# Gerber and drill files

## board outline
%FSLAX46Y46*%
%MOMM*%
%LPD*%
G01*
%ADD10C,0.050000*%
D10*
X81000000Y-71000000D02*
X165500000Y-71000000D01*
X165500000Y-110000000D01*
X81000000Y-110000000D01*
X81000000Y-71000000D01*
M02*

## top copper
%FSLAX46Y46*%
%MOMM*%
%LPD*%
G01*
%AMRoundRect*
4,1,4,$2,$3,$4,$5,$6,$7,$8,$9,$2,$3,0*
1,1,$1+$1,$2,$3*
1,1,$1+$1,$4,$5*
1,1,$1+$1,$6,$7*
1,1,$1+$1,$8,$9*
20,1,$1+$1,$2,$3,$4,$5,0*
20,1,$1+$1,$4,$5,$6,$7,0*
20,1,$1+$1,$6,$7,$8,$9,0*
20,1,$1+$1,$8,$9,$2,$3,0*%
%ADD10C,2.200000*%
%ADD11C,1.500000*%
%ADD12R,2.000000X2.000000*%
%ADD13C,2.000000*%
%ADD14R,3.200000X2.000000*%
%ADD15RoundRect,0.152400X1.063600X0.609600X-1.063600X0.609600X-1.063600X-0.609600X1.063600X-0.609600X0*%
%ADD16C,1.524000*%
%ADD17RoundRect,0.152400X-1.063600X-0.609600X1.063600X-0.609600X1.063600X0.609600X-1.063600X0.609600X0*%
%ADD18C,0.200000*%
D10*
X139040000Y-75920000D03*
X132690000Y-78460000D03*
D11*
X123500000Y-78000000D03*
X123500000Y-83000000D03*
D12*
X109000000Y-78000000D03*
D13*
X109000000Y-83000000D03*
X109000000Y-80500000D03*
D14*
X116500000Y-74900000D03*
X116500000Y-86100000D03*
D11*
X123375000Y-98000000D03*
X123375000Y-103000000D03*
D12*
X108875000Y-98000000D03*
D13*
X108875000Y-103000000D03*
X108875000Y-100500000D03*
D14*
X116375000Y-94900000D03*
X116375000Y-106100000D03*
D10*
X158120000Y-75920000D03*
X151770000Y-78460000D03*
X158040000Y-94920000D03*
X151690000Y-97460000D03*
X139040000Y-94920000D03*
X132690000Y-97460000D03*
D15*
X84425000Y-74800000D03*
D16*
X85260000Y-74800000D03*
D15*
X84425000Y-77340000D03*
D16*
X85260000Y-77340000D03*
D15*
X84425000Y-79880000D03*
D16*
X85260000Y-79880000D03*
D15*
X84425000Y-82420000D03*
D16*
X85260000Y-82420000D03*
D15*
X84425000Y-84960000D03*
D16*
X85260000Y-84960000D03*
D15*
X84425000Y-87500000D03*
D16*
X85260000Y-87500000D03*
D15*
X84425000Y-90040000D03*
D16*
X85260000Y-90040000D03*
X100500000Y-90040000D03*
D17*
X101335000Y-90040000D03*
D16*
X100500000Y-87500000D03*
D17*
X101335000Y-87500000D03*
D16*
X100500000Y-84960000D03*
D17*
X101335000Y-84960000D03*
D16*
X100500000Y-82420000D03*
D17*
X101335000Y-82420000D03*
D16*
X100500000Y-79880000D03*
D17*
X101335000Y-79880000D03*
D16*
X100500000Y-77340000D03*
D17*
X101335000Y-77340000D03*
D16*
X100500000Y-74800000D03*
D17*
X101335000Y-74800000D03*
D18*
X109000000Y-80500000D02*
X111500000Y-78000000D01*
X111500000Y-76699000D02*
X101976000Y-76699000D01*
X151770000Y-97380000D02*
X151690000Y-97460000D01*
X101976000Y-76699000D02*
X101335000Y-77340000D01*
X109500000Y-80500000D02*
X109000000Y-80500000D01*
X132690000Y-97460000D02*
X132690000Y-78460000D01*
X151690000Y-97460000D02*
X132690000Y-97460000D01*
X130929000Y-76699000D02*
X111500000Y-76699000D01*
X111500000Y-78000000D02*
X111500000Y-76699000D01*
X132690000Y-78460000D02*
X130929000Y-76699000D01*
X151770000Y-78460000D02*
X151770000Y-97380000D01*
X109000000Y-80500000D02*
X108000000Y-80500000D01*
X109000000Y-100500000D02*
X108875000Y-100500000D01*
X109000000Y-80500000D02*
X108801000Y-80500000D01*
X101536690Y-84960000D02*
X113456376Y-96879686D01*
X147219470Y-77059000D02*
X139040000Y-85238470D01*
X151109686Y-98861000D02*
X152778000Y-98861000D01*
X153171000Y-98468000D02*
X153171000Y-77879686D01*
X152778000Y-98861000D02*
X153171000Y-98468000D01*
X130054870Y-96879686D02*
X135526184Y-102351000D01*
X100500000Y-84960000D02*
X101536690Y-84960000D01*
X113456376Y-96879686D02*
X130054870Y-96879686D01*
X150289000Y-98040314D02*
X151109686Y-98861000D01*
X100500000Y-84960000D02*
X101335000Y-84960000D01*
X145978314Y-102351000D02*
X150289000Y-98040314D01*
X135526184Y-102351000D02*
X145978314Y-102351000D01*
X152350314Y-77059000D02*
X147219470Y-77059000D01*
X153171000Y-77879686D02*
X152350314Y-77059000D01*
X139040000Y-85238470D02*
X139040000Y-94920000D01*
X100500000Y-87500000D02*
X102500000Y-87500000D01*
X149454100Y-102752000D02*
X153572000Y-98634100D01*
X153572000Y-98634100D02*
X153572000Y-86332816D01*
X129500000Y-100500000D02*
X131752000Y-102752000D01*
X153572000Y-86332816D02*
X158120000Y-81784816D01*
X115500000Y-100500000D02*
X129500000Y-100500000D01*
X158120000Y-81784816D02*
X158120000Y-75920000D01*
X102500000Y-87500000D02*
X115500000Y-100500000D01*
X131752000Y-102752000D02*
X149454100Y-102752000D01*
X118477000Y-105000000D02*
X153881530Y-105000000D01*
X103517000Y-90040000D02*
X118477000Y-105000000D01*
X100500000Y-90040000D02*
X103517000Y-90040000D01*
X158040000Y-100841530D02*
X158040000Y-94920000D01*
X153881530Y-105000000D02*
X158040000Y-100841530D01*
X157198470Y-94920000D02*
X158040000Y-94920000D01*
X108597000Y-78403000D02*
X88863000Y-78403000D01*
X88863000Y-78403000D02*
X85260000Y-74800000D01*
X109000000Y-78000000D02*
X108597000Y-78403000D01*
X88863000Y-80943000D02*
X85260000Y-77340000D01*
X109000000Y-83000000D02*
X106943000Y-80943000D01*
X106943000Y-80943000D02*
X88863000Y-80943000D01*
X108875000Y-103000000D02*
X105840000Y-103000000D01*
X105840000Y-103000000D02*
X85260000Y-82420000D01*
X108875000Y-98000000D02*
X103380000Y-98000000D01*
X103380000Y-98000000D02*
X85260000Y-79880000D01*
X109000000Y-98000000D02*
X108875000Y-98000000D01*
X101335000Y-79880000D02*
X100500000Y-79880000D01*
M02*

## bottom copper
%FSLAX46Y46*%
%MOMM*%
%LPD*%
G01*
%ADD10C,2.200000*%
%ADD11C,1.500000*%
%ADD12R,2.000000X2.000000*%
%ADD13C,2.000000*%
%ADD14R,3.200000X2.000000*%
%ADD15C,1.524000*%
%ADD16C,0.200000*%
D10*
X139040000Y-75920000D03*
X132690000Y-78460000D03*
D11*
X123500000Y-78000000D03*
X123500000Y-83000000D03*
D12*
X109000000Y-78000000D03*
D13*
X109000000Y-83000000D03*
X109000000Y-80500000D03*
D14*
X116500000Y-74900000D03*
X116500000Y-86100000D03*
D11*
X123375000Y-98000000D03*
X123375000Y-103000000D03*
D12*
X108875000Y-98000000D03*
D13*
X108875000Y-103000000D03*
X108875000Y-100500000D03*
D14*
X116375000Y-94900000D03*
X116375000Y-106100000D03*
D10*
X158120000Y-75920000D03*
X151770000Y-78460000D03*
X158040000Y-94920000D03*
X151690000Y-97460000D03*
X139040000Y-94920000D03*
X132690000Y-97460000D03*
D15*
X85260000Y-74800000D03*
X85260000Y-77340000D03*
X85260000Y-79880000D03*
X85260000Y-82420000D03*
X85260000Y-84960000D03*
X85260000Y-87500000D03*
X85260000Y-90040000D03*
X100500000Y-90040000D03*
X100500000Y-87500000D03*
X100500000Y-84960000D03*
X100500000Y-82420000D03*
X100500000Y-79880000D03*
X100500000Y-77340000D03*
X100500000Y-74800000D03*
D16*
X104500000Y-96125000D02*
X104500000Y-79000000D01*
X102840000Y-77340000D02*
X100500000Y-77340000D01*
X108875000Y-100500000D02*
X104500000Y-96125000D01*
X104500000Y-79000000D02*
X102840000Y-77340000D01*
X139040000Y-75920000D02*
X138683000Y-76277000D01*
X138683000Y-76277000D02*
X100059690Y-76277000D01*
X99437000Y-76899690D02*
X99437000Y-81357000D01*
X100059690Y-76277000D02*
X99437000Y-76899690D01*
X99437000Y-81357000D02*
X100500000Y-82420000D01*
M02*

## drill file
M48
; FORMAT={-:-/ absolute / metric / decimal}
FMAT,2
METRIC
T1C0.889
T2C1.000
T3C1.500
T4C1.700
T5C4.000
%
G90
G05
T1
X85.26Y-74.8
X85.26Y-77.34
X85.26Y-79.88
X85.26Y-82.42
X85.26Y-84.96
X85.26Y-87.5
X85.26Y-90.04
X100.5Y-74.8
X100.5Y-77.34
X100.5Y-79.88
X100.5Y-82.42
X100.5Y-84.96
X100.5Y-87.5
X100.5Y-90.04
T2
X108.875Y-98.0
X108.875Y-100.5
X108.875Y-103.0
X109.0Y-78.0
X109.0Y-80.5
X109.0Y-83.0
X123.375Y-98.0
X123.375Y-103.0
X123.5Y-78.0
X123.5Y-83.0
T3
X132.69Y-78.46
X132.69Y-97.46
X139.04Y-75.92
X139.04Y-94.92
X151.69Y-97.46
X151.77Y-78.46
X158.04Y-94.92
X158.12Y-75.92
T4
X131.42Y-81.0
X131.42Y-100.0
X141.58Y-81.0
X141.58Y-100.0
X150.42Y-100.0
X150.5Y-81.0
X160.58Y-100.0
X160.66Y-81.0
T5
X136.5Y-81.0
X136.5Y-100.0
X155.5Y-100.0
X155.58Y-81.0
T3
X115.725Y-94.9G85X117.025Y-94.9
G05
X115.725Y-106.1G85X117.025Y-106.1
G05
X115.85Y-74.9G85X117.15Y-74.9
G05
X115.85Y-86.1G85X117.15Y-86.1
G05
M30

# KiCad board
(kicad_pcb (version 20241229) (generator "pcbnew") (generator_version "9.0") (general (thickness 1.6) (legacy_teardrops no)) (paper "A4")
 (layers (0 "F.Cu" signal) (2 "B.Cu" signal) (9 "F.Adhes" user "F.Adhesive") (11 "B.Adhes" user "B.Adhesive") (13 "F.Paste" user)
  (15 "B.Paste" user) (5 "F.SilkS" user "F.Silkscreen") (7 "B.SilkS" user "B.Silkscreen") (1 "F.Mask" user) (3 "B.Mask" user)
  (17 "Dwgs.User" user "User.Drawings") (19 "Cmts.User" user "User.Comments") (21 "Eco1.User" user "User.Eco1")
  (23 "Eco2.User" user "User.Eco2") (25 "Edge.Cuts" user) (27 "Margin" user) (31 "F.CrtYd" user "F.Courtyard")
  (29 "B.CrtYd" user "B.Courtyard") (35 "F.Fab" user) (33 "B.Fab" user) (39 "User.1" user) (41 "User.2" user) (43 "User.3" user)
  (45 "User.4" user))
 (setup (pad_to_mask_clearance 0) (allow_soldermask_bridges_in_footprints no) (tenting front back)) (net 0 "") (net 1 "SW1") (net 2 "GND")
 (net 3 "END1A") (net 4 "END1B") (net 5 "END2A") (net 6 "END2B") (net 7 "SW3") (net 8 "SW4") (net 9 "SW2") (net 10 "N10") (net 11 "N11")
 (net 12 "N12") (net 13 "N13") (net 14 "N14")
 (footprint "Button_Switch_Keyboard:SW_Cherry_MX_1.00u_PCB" (layer "F.Cu") (at 139.04 75.92)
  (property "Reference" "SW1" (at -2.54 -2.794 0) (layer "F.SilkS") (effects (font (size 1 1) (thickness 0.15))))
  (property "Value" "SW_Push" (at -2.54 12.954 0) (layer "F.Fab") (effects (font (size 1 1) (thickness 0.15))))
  (pad "" np_thru_hole circle (at -7.62 5.08) (size 1.7 1.7) (drill 1.7) (layers "*.Cu" "*.Mask"))
  (pad "" np_thru_hole circle (at -2.54 5.08) (size 4 4) (drill 4) (layers "*.Cu" "*.Mask"))
  (pad "" np_thru_hole circle (at 2.54 5.08) (size 1.7 1.7) (drill 1.7) (layers "*.Cu" "*.Mask"))
  (pad "1" thru_hole circle (at 0 0) (size 2.2 2.2) (drill 1.5) (layers "*.Cu" "*.Mask") (remove_unused_layers no) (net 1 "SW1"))
  (pad "2" thru_hole circle (at -6.35 2.54) (size 2.2 2.2) (drill 1.5) (layers "*.Cu" "*.Mask") (remove_unused_layers no) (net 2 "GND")))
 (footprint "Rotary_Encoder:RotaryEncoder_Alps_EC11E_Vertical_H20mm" (layer "F.Cu") (at 109 78)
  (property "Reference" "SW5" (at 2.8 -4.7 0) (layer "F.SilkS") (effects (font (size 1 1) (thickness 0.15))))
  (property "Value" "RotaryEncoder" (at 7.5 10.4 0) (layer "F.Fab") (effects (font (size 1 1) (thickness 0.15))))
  (pad "" thru_hole circle (at 14.5 0) (size 1.5 1.5) (drill 1) (layers "*.Cu" "*.Mask") (remove_unused_layers no))
  (pad "" thru_hole circle (at 14.5 5) (size 1.5 1.5) (drill 1) (layers "*.Cu" "*.Mask") (remove_unused_layers no))
  (pad "A" thru_hole rect (at 0 0) (size 2 2) (drill 1) (layers "*.Cu" "*.Mask") (remove_unused_layers no) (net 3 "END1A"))
  (pad "B" thru_hole circle (at 0 5) (size 2 2) (drill 1) (layers "*.Cu" "*.Mask") (remove_unused_layers no) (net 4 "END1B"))
  (pad "C" thru_hole circle (at 0 2.5) (size 2 2) (drill 1) (layers "*.Cu" "*.Mask") (remove_unused_layers no) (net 2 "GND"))
  (pad "MP" thru_hole rect (at 7.5 -3.1) (size 3.2 2) (drill oval 2.8 1.5) (layers "*.Cu" "*.Mask") (remove_unused_layers no))
  (pad "MP" thru_hole rect (at 7.5 8.1) (size 3.2 2) (drill oval 2.8 1.5) (layers "*.Cu" "*.Mask") (remove_unused_layers no)))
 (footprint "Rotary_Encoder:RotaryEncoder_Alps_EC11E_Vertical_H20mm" (layer "F.Cu") (at 108.875 98)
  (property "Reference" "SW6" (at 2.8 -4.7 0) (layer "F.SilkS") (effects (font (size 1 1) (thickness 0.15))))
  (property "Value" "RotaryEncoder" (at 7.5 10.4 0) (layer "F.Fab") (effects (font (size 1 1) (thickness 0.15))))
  (pad "" thru_hole circle (at 14.5 0) (size 1.5 1.5) (drill 1) (layers "*.Cu" "*.Mask") (remove_unused_layers no))
  (pad "" thru_hole circle (at 14.5 5) (size 1.5 1.5) (drill 1) (layers "*.Cu" "*.Mask") (remove_unused_layers no))
  (pad "A" thru_hole rect (at 0 0) (size 2 2) (drill 1) (layers "*.Cu" "*.Mask") (remove_unused_layers no) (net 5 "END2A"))
  (pad "B" thru_hole circle (at 0 5) (size 2 2) (drill 1) (layers "*.Cu" "*.Mask") (remove_unused_layers no) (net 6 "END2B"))
  (pad "C" thru_hole circle (at 0 2.5) (size 2 2) (drill 1) (layers "*.Cu" "*.Mask") (remove_unused_layers no) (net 2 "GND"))
  (pad "MP" thru_hole rect (at 7.5 -3.1) (size 3.2 2) (drill oval 2.8 1.5) (layers "*.Cu" "*.Mask") (remove_unused_layers no))
  (pad "MP" thru_hole rect (at 7.5 8.1) (size 3.2 2) (drill oval 2.8 1.5) (layers "*.Cu" "*.Mask") (remove_unused_layers no)))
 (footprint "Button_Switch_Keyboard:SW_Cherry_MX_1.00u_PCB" (layer "F.Cu") (at 158.12 75.92)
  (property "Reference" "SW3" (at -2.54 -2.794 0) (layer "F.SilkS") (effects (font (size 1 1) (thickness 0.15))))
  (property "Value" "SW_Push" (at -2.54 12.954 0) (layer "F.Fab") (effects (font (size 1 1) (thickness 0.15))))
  (pad "" np_thru_hole circle (at -7.62 5.08) (size 1.7 1.7) (drill 1.7) (layers "*.Cu" "*.Mask"))
  (pad "" np_thru_hole circle (at -2.54 5.08) (size 4 4) (drill 4) (layers "*.Cu" "*.Mask"))
  (pad "" np_thru_hole circle (at 2.54 5.08) (size 1.7 1.7) (drill 1.7) (layers "*.Cu" "*.Mask"))
  (pad "1" thru_hole circle (at 0 0) (size 2.2 2.2) (drill 1.5) (layers "*.Cu" "*.Mask") (remove_unused_layers no) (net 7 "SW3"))
  (pad "2" thru_hole circle (at -6.35 2.54) (size 2.2 2.2) (drill 1.5) (layers "*.Cu" "*.Mask") (remove_unused_layers no) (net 2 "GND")))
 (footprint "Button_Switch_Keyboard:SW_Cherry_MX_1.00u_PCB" (layer "F.Cu") (at 158.04 94.92)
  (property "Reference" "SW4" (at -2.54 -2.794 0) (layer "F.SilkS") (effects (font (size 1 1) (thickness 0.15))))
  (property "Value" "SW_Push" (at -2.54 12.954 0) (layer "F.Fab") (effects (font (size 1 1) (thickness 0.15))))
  (pad "" np_thru_hole circle (at -7.62 5.08) (size 1.7 1.7) (drill 1.7) (layers "*.Cu" "*.Mask"))
  (pad "" np_thru_hole circle (at -2.54 5.08) (size 4 4) (drill 4) (layers "*.Cu" "*.Mask"))
  (pad "" np_thru_hole circle (at 2.54 5.08) (size 1.7 1.7) (drill 1.7) (layers "*.Cu" "*.Mask"))
  (pad "1" thru_hole circle (at 0 0) (size 2.2 2.2) (drill 1.5) (layers "*.Cu" "*.Mask") (remove_unused_layers no) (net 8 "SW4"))
  (pad "2" thru_hole circle (at -6.35 2.54) (size 2.2 2.2) (drill 1.5) (layers "*.Cu" "*.Mask") (remove_unused_layers no) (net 2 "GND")))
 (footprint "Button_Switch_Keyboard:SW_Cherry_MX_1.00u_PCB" (layer "F.Cu") (at 139.04 94.92)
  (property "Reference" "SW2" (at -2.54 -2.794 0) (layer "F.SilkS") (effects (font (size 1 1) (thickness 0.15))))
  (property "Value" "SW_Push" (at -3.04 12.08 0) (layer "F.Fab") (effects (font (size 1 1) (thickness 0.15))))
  (pad "" np_thru_hole circle (at -7.62 5.08) (size 1.7 1.7) (drill 1.7) (layers "*.Cu" "*.Mask"))
  (pad "" np_thru_hole circle (at -2.54 5.08) (size 4 4) (drill 4) (layers "*.Cu" "*.Mask"))
  (pad "" np_thru_hole circle (at 2.54 5.08) (size 1.7 1.7) (drill 1.7) (layers "*.Cu" "*.Mask"))
  (pad "1" thru_hole circle (at 0 0) (size 2.2 2.2) (drill 1.5) (layers "*.Cu" "*.Mask") (remove_unused_layers no) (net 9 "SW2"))
  (pad "2" thru_hole circle (at -6.35 2.54) (size 2.2 2.2) (drill 1.5) (layers "*.Cu" "*.Mask") (remove_unused_layers no) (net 2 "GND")))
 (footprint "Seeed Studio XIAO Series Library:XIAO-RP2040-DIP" (layer "F.Cu") (at 92.88 82.42)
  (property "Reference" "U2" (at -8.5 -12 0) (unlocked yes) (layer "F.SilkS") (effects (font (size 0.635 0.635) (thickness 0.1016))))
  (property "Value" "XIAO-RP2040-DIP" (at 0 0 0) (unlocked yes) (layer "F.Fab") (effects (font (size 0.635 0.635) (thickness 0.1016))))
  (pad "1" smd roundrect (at -8.455 -7.62 180) (size 2.432 1.524) (layers "F.Cu" "F.Mask") (roundrect_rratio 0.1) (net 3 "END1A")
   (thermal_bridge_angle 45))
  (pad "1" thru_hole circle (at -7.62 -7.62 180) (size 1.524 1.524) (drill 0.889) (layers "*.Cu" "*.Mask") (remove_unused_layers no)
   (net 3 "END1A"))
  (pad "2" smd roundrect (at -8.455 -5.08 180) (size 2.432 1.524) (layers "F.Cu" "F.Mask") (roundrect_rratio 0.1) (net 4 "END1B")
   (thermal_bridge_angle 45))
  (pad "2" thru_hole circle (at -7.62 -5.08 180) (size 1.524 1.524) (drill 0.889) (layers "*.Cu" "*.Mask") (remove_unused_layers no)
   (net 4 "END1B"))
  (pad "3" smd roundrect (at -8.455 -2.54 180) (size 2.432 1.524) (layers "F.Cu" "F.Mask") (roundrect_rratio 0.1) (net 5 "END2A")
   (thermal_bridge_angle 45))
  (pad "3" thru_hole circle (at -7.62 -2.54 180) (size 1.524 1.524) (drill 0.889) (layers "*.Cu" "*.Mask") (remove_unused_layers no)
   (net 5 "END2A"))
  (pad "4" smd roundrect (at -8.455 0 180) (size 2.432 1.524) (layers "F.Cu" "F.Mask") (roundrect_rratio 0.1) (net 6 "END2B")
   (thermal_bridge_angle 45))
  (pad "4" thru_hole circle (at -7.62 0 180) (size 1.524 1.524) (drill 0.889) (layers "*.Cu" "*.Mask") (remove_unused_layers no)
   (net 6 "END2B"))
  (pad "5" smd roundrect (at -8.455 2.54 180) (size 2.432 1.524) (layers "F.Cu" "F.Mask") (roundrect_rratio 0.1) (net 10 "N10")
   (thermal_bridge_angle 45))
  (pad "5" thru_hole circle (at -7.62 2.54 180) (size 1.524 1.524) (drill 0.889) (layers "*.Cu" "*.Mask") (remove_unused_layers no)
   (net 10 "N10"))
  (pad "6" smd roundrect (at -8.455 5.08 180) (size 2.432 1.524) (layers "F.Cu" "F.Mask") (roundrect_rratio 0.1) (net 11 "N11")
   (thermal_bridge_angle 45))
  (pad "6" thru_hole circle (at -7.62 5.08 180) (size 1.524 1.524) (drill 0.889) (layers "*.Cu" "*.Mask") (remove_unused_layers no)
   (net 11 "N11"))
  (pad "7" smd roundrect (at -8.455 7.62 180) (size 2.432 1.524) (layers "F.Cu" "F.Mask") (roundrect_rratio 0.1) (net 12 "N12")
   (thermal_bridge_angle 45))
  (pad "7" thru_hole circle (at -7.62 7.62 180) (size 1.524 1.524) (drill 0.889) (layers "*.Cu" "*.Mask") (remove_unused_layers no)
   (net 12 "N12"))
  (pad "8" thru_hole circle (at 7.62 7.62) (size 1.524 1.524) (drill 0.889) (layers "*.Cu" "*.Mask") (remove_unused_layers no) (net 8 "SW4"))
  (pad "8" smd roundrect (at 8.455 7.62) (size 2.432 1.524) (layers "F.Cu" "F.Mask") (roundrect_rratio 0.1) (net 8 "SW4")
   (thermal_bridge_angle 45))
  (pad "9" thru_hole circle (at 7.62 5.08) (size 1.524 1.524) (drill 0.889) (layers "*.Cu" "*.Mask") (remove_unused_layers no) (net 7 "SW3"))
  (pad "9" smd roundrect (at 8.455 5.08) (size 2.432 1.524) (layers "F.Cu" "F.Mask") (roundrect_rratio 0.1) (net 7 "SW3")
   (thermal_bridge_angle 45))
  (pad "10" thru_hole circle (at 7.62 2.54) (size 1.524 1.524) (drill 0.889) (layers "*.Cu" "*.Mask") (remove_unused_layers no)
   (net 9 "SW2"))
  (pad "10" smd roundrect (at 8.455 2.54) (size 2.432 1.524) (layers "F.Cu" "F.Mask") (roundrect_rratio 0.1) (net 9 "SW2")
   (thermal_bridge_angle 45))
  (pad "11" thru_hole circle (at 7.62 0) (size 1.524 1.524) (drill 0.889) (layers "*.Cu" "*.Mask") (remove_unused_layers no) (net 1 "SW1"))
  (pad "11" smd roundrect (at 8.455 0) (size 2.432 1.524) (layers "F.Cu" "F.Mask") (roundrect_rratio 0.1) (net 1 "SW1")
   (thermal_bridge_angle 45))
  (pad "12" thru_hole circle (at 7.62 -2.54) (size 1.524 1.524) (drill 0.889) (layers "*.Cu" "*.Mask") (remove_unused_layers no)
   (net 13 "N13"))
  (pad "12" smd roundrect (at 8.455 -2.54) (size 2.432 1.524) (layers "F.Cu" "F.Mask") (roundrect_rratio 0.1) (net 13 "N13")
   (thermal_bridge_angle 45))
  (pad "13" thru_hole circle (at 7.62 -5.08) (size 1.524 1.524) (drill 0.889) (layers "*.Cu" "*.Mask") (remove_unused_layers no)
   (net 2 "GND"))
  (pad "13" smd roundrect (at 8.455 -5.08) (size 2.432 1.524) (layers "F.Cu" "F.Mask") (roundrect_rratio 0.1) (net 2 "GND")
   (thermal_bridge_angle 45))
  (pad "14" thru_hole circle (at 7.62 -7.62) (size 1.524 1.524) (drill 0.889) (layers "*.Cu" "*.Mask") (remove_unused_layers no)
   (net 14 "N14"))
  (pad "14" smd roundrect (at 8.455 -7.62) (size 2.432 1.524) (layers "F.Cu" "F.Mask") (roundrect_rratio 0.1) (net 14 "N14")
   (thermal_bridge_angle 45)))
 (gr_rect (start 81 71) (end 165.5 110) (stroke (width 0.05) (type default)) (fill no) (layer "Edge.Cuts"))
 (segment (start 109 80.5) (end 111.5 78) (width 0.2) (layer "F.Cu") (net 2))
 (segment (start 111.5 76.699) (end 101.976 76.699) (width 0.2) (layer "F.Cu") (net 2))
 (segment (start 151.77 97.38) (end 151.69 97.46) (width 0.2) (layer "F.Cu") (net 2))
 (segment (start 101.976 76.699) (end 101.335 77.34) (width 0.2) (layer "F.Cu") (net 2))
 (segment (start 109.5 80.5) (end 109 80.5) (width 0.2) (layer "F.Cu") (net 2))
 (segment (start 132.69 97.46) (end 132.69 78.46) (width 0.2) (layer "F.Cu") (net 2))
 (segment (start 151.69 97.46) (end 132.69 97.46) (width 0.2) (layer "F.Cu") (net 2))
 (segment (start 130.929 76.699) (end 111.5 76.699) (width 0.2) (layer "F.Cu") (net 2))
 (segment (start 111.5 78) (end 111.5 76.699) (width 0.2) (layer "F.Cu") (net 2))
 (segment (start 132.69 78.46) (end 130.929 76.699) (width 0.2) (layer "F.Cu") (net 2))
 (segment (start 151.77 78.46) (end 151.77 97.38) (width 0.2) (layer "F.Cu") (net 2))
 (segment (start 109 80.5) (end 108 80.5) (width 0.2) (layer "F.Cu") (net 2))
 (segment (start 109 100.5) (end 108.875 100.5) (width 0.2) (layer "F.Cu") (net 2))
 (segment (start 109 80.5) (end 108.801 80.5) (width 0.2) (layer "F.Cu") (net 2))
 (segment (start 104.5 96.125) (end 104.5 79) (width 0.2) (layer "B.Cu") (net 2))
 (segment (start 102.84 77.34) (end 100.5 77.34) (width 0.2) (layer "B.Cu") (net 2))
 (segment (start 108.875 100.5) (end 104.5 96.125) (width 0.2) (layer "B.Cu") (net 2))
 (segment (start 104.5 79) (end 102.84 77.34) (width 0.2) (layer "B.Cu") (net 2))
 (segment (start 139.04 75.92) (end 138.683 76.277) (width 0.2) (layer "B.Cu") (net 1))
 (segment (start 138.683 76.277) (end 100.05969 76.277) (width 0.2) (layer "B.Cu") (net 1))
 (segment (start 99.437 76.89969) (end 99.437 81.357) (width 0.2) (layer "B.Cu") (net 1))
 (segment (start 100.05969 76.277) (end 99.437 76.89969) (width 0.2) (layer "B.Cu") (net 1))
 (segment (start 99.437 81.357) (end 100.5 82.42) (width 0.2) (layer "B.Cu") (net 1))
 (segment (start 101.53669 84.96) (end 113.456376 96.879686) (width 0.2) (layer "F.Cu") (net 9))
 (segment (start 147.21947 77.059) (end 139.04 85.23847) (width 0.2) (layer "F.Cu") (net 9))
 (segment (start 151.109686 98.861) (end 152.778 98.861) (width 0.2) (layer "F.Cu") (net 9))
 (segment (start 153.171 98.468) (end 153.171 77.879686) (width 0.2) (layer "F.Cu") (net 9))
 (segment (start 152.778 98.861) (end 153.171 98.468) (width 0.2) (layer "F.Cu") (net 9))
 (segment (start 130.05487 96.879686) (end 135.526184 102.351) (width 0.2) (layer "F.Cu") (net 9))
 (segment (start 100.5 84.96) (end 101.53669 84.96) (width 0.2) (layer "F.Cu") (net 9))
 (segment (start 113.456376 96.879686) (end 130.05487 96.879686) (width 0.2) (layer "F.Cu") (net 9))
 (segment (start 150.289 98.040314) (end 151.109686 98.861) (width 0.2) (layer "F.Cu") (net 9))
 (segment (start 100.5 84.96) (end 101.335 84.96) (width 0.2) (layer "F.Cu") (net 9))
 (segment (start 145.978314 102.351) (end 150.289 98.040314) (width 0.2) (layer "F.Cu") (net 9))
 (segment (start 135.526184 102.351) (end 145.978314 102.351) (width 0.2) (layer "F.Cu") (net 9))
 (segment (start 152.350314 77.059) (end 147.21947 77.059) (width 0.2) (layer "F.Cu") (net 9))
 (segment (start 153.171 77.879686) (end 152.350314 77.059) (width 0.2) (layer "F.Cu") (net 9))
 (segment (start 139.04 85.23847) (end 139.04 94.92) (width 0.2) (layer "F.Cu") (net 9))
 (segment (start 100.5 87.5) (end 102.5 87.5) (width 0.2) (layer "F.Cu") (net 7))
 (segment (start 149.4541 102.752) (end 153.572 98.6341) (width 0.2) (layer "F.Cu") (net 7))
 (segment (start 153.572 98.6341) (end 153.572 86.332816) (width 0.2) (layer "F.Cu") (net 7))
 (segment (start 129.5 100.5) (end 131.752 102.752) (width 0.2) (layer "F.Cu") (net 7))
 (segment (start 153.572 86.332816) (end 158.12 81.784816) (width 0.2) (layer "F.Cu") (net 7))
 (segment (start 115.5 100.5) (end 129.5 100.5) (width 0.2) (layer "F.Cu") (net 7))
 (segment (start 158.12 81.784816) (end 158.12 75.92) (width 0.2) (layer "F.Cu") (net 7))
 (segment (start 102.5 87.5) (end 115.5 100.5) (width 0.2) (layer "F.Cu") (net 7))
 (segment (start 131.752 102.752) (end 149.4541 102.752) (width 0.2) (layer "F.Cu") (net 7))
 (segment (start 118.477 105) (end 153.88153 105) (width 0.2) (layer "F.Cu") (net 8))
 (segment (start 103.517 90.04) (end 118.477 105) (width 0.2) (layer "F.Cu") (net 8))
 (segment (start 100.5 90.04) (end 103.517 90.04) (width 0.2) (layer "F.Cu") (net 8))
 (segment (start 158.04 100.84153) (end 158.04 94.92) (width 0.2) (layer "F.Cu") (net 8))
 (segment (start 153.88153 105) (end 158.04 100.84153) (width 0.2) (layer "F.Cu") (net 8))
 (segment (start 157.19847 94.92) (end 158.04 94.92) (width 0.2) (layer "F.Cu") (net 8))
 (segment (start 108.597 78.403) (end 88.863 78.403) (width 0.2) (layer "F.Cu") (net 3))
 (segment (start 88.863 78.403) (end 85.26 74.8) (width 0.2) (layer "F.Cu") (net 3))
 (segment (start 109 78) (end 108.597 78.403) (width 0.2) (layer "F.Cu") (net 3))
 (segment (start 88.863 80.943) (end 85.26 77.34) (width 0.2) (layer "F.Cu") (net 4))
 (segment (start 109 83) (end 106.943 80.943) (width 0.2) (layer "F.Cu") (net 4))
 (segment (start 106.943 80.943) (end 88.863 80.943) (width 0.2) (layer "F.Cu") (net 4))
 (segment (start 108.875 103) (end 105.84 103) (width 0.2) (layer "F.Cu") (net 6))
 (segment (start 105.84 103) (end 85.26 82.42) (width 0.2) (layer "F.Cu") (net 6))
 (segment (start 108.875 98) (end 103.38 98) (width 0.2) (layer "F.Cu") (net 5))
 (segment (start 103.38 98) (end 85.26 79.88) (width 0.2) (layer "F.Cu") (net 5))
 (segment (start 109 98) (end 108.875 98) (width 0.2) (layer "F.Cu") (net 5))
 (segment (start 101.335 79.88) (end 100.5 79.88) (width 0.2) (layer "F.Cu") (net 13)))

